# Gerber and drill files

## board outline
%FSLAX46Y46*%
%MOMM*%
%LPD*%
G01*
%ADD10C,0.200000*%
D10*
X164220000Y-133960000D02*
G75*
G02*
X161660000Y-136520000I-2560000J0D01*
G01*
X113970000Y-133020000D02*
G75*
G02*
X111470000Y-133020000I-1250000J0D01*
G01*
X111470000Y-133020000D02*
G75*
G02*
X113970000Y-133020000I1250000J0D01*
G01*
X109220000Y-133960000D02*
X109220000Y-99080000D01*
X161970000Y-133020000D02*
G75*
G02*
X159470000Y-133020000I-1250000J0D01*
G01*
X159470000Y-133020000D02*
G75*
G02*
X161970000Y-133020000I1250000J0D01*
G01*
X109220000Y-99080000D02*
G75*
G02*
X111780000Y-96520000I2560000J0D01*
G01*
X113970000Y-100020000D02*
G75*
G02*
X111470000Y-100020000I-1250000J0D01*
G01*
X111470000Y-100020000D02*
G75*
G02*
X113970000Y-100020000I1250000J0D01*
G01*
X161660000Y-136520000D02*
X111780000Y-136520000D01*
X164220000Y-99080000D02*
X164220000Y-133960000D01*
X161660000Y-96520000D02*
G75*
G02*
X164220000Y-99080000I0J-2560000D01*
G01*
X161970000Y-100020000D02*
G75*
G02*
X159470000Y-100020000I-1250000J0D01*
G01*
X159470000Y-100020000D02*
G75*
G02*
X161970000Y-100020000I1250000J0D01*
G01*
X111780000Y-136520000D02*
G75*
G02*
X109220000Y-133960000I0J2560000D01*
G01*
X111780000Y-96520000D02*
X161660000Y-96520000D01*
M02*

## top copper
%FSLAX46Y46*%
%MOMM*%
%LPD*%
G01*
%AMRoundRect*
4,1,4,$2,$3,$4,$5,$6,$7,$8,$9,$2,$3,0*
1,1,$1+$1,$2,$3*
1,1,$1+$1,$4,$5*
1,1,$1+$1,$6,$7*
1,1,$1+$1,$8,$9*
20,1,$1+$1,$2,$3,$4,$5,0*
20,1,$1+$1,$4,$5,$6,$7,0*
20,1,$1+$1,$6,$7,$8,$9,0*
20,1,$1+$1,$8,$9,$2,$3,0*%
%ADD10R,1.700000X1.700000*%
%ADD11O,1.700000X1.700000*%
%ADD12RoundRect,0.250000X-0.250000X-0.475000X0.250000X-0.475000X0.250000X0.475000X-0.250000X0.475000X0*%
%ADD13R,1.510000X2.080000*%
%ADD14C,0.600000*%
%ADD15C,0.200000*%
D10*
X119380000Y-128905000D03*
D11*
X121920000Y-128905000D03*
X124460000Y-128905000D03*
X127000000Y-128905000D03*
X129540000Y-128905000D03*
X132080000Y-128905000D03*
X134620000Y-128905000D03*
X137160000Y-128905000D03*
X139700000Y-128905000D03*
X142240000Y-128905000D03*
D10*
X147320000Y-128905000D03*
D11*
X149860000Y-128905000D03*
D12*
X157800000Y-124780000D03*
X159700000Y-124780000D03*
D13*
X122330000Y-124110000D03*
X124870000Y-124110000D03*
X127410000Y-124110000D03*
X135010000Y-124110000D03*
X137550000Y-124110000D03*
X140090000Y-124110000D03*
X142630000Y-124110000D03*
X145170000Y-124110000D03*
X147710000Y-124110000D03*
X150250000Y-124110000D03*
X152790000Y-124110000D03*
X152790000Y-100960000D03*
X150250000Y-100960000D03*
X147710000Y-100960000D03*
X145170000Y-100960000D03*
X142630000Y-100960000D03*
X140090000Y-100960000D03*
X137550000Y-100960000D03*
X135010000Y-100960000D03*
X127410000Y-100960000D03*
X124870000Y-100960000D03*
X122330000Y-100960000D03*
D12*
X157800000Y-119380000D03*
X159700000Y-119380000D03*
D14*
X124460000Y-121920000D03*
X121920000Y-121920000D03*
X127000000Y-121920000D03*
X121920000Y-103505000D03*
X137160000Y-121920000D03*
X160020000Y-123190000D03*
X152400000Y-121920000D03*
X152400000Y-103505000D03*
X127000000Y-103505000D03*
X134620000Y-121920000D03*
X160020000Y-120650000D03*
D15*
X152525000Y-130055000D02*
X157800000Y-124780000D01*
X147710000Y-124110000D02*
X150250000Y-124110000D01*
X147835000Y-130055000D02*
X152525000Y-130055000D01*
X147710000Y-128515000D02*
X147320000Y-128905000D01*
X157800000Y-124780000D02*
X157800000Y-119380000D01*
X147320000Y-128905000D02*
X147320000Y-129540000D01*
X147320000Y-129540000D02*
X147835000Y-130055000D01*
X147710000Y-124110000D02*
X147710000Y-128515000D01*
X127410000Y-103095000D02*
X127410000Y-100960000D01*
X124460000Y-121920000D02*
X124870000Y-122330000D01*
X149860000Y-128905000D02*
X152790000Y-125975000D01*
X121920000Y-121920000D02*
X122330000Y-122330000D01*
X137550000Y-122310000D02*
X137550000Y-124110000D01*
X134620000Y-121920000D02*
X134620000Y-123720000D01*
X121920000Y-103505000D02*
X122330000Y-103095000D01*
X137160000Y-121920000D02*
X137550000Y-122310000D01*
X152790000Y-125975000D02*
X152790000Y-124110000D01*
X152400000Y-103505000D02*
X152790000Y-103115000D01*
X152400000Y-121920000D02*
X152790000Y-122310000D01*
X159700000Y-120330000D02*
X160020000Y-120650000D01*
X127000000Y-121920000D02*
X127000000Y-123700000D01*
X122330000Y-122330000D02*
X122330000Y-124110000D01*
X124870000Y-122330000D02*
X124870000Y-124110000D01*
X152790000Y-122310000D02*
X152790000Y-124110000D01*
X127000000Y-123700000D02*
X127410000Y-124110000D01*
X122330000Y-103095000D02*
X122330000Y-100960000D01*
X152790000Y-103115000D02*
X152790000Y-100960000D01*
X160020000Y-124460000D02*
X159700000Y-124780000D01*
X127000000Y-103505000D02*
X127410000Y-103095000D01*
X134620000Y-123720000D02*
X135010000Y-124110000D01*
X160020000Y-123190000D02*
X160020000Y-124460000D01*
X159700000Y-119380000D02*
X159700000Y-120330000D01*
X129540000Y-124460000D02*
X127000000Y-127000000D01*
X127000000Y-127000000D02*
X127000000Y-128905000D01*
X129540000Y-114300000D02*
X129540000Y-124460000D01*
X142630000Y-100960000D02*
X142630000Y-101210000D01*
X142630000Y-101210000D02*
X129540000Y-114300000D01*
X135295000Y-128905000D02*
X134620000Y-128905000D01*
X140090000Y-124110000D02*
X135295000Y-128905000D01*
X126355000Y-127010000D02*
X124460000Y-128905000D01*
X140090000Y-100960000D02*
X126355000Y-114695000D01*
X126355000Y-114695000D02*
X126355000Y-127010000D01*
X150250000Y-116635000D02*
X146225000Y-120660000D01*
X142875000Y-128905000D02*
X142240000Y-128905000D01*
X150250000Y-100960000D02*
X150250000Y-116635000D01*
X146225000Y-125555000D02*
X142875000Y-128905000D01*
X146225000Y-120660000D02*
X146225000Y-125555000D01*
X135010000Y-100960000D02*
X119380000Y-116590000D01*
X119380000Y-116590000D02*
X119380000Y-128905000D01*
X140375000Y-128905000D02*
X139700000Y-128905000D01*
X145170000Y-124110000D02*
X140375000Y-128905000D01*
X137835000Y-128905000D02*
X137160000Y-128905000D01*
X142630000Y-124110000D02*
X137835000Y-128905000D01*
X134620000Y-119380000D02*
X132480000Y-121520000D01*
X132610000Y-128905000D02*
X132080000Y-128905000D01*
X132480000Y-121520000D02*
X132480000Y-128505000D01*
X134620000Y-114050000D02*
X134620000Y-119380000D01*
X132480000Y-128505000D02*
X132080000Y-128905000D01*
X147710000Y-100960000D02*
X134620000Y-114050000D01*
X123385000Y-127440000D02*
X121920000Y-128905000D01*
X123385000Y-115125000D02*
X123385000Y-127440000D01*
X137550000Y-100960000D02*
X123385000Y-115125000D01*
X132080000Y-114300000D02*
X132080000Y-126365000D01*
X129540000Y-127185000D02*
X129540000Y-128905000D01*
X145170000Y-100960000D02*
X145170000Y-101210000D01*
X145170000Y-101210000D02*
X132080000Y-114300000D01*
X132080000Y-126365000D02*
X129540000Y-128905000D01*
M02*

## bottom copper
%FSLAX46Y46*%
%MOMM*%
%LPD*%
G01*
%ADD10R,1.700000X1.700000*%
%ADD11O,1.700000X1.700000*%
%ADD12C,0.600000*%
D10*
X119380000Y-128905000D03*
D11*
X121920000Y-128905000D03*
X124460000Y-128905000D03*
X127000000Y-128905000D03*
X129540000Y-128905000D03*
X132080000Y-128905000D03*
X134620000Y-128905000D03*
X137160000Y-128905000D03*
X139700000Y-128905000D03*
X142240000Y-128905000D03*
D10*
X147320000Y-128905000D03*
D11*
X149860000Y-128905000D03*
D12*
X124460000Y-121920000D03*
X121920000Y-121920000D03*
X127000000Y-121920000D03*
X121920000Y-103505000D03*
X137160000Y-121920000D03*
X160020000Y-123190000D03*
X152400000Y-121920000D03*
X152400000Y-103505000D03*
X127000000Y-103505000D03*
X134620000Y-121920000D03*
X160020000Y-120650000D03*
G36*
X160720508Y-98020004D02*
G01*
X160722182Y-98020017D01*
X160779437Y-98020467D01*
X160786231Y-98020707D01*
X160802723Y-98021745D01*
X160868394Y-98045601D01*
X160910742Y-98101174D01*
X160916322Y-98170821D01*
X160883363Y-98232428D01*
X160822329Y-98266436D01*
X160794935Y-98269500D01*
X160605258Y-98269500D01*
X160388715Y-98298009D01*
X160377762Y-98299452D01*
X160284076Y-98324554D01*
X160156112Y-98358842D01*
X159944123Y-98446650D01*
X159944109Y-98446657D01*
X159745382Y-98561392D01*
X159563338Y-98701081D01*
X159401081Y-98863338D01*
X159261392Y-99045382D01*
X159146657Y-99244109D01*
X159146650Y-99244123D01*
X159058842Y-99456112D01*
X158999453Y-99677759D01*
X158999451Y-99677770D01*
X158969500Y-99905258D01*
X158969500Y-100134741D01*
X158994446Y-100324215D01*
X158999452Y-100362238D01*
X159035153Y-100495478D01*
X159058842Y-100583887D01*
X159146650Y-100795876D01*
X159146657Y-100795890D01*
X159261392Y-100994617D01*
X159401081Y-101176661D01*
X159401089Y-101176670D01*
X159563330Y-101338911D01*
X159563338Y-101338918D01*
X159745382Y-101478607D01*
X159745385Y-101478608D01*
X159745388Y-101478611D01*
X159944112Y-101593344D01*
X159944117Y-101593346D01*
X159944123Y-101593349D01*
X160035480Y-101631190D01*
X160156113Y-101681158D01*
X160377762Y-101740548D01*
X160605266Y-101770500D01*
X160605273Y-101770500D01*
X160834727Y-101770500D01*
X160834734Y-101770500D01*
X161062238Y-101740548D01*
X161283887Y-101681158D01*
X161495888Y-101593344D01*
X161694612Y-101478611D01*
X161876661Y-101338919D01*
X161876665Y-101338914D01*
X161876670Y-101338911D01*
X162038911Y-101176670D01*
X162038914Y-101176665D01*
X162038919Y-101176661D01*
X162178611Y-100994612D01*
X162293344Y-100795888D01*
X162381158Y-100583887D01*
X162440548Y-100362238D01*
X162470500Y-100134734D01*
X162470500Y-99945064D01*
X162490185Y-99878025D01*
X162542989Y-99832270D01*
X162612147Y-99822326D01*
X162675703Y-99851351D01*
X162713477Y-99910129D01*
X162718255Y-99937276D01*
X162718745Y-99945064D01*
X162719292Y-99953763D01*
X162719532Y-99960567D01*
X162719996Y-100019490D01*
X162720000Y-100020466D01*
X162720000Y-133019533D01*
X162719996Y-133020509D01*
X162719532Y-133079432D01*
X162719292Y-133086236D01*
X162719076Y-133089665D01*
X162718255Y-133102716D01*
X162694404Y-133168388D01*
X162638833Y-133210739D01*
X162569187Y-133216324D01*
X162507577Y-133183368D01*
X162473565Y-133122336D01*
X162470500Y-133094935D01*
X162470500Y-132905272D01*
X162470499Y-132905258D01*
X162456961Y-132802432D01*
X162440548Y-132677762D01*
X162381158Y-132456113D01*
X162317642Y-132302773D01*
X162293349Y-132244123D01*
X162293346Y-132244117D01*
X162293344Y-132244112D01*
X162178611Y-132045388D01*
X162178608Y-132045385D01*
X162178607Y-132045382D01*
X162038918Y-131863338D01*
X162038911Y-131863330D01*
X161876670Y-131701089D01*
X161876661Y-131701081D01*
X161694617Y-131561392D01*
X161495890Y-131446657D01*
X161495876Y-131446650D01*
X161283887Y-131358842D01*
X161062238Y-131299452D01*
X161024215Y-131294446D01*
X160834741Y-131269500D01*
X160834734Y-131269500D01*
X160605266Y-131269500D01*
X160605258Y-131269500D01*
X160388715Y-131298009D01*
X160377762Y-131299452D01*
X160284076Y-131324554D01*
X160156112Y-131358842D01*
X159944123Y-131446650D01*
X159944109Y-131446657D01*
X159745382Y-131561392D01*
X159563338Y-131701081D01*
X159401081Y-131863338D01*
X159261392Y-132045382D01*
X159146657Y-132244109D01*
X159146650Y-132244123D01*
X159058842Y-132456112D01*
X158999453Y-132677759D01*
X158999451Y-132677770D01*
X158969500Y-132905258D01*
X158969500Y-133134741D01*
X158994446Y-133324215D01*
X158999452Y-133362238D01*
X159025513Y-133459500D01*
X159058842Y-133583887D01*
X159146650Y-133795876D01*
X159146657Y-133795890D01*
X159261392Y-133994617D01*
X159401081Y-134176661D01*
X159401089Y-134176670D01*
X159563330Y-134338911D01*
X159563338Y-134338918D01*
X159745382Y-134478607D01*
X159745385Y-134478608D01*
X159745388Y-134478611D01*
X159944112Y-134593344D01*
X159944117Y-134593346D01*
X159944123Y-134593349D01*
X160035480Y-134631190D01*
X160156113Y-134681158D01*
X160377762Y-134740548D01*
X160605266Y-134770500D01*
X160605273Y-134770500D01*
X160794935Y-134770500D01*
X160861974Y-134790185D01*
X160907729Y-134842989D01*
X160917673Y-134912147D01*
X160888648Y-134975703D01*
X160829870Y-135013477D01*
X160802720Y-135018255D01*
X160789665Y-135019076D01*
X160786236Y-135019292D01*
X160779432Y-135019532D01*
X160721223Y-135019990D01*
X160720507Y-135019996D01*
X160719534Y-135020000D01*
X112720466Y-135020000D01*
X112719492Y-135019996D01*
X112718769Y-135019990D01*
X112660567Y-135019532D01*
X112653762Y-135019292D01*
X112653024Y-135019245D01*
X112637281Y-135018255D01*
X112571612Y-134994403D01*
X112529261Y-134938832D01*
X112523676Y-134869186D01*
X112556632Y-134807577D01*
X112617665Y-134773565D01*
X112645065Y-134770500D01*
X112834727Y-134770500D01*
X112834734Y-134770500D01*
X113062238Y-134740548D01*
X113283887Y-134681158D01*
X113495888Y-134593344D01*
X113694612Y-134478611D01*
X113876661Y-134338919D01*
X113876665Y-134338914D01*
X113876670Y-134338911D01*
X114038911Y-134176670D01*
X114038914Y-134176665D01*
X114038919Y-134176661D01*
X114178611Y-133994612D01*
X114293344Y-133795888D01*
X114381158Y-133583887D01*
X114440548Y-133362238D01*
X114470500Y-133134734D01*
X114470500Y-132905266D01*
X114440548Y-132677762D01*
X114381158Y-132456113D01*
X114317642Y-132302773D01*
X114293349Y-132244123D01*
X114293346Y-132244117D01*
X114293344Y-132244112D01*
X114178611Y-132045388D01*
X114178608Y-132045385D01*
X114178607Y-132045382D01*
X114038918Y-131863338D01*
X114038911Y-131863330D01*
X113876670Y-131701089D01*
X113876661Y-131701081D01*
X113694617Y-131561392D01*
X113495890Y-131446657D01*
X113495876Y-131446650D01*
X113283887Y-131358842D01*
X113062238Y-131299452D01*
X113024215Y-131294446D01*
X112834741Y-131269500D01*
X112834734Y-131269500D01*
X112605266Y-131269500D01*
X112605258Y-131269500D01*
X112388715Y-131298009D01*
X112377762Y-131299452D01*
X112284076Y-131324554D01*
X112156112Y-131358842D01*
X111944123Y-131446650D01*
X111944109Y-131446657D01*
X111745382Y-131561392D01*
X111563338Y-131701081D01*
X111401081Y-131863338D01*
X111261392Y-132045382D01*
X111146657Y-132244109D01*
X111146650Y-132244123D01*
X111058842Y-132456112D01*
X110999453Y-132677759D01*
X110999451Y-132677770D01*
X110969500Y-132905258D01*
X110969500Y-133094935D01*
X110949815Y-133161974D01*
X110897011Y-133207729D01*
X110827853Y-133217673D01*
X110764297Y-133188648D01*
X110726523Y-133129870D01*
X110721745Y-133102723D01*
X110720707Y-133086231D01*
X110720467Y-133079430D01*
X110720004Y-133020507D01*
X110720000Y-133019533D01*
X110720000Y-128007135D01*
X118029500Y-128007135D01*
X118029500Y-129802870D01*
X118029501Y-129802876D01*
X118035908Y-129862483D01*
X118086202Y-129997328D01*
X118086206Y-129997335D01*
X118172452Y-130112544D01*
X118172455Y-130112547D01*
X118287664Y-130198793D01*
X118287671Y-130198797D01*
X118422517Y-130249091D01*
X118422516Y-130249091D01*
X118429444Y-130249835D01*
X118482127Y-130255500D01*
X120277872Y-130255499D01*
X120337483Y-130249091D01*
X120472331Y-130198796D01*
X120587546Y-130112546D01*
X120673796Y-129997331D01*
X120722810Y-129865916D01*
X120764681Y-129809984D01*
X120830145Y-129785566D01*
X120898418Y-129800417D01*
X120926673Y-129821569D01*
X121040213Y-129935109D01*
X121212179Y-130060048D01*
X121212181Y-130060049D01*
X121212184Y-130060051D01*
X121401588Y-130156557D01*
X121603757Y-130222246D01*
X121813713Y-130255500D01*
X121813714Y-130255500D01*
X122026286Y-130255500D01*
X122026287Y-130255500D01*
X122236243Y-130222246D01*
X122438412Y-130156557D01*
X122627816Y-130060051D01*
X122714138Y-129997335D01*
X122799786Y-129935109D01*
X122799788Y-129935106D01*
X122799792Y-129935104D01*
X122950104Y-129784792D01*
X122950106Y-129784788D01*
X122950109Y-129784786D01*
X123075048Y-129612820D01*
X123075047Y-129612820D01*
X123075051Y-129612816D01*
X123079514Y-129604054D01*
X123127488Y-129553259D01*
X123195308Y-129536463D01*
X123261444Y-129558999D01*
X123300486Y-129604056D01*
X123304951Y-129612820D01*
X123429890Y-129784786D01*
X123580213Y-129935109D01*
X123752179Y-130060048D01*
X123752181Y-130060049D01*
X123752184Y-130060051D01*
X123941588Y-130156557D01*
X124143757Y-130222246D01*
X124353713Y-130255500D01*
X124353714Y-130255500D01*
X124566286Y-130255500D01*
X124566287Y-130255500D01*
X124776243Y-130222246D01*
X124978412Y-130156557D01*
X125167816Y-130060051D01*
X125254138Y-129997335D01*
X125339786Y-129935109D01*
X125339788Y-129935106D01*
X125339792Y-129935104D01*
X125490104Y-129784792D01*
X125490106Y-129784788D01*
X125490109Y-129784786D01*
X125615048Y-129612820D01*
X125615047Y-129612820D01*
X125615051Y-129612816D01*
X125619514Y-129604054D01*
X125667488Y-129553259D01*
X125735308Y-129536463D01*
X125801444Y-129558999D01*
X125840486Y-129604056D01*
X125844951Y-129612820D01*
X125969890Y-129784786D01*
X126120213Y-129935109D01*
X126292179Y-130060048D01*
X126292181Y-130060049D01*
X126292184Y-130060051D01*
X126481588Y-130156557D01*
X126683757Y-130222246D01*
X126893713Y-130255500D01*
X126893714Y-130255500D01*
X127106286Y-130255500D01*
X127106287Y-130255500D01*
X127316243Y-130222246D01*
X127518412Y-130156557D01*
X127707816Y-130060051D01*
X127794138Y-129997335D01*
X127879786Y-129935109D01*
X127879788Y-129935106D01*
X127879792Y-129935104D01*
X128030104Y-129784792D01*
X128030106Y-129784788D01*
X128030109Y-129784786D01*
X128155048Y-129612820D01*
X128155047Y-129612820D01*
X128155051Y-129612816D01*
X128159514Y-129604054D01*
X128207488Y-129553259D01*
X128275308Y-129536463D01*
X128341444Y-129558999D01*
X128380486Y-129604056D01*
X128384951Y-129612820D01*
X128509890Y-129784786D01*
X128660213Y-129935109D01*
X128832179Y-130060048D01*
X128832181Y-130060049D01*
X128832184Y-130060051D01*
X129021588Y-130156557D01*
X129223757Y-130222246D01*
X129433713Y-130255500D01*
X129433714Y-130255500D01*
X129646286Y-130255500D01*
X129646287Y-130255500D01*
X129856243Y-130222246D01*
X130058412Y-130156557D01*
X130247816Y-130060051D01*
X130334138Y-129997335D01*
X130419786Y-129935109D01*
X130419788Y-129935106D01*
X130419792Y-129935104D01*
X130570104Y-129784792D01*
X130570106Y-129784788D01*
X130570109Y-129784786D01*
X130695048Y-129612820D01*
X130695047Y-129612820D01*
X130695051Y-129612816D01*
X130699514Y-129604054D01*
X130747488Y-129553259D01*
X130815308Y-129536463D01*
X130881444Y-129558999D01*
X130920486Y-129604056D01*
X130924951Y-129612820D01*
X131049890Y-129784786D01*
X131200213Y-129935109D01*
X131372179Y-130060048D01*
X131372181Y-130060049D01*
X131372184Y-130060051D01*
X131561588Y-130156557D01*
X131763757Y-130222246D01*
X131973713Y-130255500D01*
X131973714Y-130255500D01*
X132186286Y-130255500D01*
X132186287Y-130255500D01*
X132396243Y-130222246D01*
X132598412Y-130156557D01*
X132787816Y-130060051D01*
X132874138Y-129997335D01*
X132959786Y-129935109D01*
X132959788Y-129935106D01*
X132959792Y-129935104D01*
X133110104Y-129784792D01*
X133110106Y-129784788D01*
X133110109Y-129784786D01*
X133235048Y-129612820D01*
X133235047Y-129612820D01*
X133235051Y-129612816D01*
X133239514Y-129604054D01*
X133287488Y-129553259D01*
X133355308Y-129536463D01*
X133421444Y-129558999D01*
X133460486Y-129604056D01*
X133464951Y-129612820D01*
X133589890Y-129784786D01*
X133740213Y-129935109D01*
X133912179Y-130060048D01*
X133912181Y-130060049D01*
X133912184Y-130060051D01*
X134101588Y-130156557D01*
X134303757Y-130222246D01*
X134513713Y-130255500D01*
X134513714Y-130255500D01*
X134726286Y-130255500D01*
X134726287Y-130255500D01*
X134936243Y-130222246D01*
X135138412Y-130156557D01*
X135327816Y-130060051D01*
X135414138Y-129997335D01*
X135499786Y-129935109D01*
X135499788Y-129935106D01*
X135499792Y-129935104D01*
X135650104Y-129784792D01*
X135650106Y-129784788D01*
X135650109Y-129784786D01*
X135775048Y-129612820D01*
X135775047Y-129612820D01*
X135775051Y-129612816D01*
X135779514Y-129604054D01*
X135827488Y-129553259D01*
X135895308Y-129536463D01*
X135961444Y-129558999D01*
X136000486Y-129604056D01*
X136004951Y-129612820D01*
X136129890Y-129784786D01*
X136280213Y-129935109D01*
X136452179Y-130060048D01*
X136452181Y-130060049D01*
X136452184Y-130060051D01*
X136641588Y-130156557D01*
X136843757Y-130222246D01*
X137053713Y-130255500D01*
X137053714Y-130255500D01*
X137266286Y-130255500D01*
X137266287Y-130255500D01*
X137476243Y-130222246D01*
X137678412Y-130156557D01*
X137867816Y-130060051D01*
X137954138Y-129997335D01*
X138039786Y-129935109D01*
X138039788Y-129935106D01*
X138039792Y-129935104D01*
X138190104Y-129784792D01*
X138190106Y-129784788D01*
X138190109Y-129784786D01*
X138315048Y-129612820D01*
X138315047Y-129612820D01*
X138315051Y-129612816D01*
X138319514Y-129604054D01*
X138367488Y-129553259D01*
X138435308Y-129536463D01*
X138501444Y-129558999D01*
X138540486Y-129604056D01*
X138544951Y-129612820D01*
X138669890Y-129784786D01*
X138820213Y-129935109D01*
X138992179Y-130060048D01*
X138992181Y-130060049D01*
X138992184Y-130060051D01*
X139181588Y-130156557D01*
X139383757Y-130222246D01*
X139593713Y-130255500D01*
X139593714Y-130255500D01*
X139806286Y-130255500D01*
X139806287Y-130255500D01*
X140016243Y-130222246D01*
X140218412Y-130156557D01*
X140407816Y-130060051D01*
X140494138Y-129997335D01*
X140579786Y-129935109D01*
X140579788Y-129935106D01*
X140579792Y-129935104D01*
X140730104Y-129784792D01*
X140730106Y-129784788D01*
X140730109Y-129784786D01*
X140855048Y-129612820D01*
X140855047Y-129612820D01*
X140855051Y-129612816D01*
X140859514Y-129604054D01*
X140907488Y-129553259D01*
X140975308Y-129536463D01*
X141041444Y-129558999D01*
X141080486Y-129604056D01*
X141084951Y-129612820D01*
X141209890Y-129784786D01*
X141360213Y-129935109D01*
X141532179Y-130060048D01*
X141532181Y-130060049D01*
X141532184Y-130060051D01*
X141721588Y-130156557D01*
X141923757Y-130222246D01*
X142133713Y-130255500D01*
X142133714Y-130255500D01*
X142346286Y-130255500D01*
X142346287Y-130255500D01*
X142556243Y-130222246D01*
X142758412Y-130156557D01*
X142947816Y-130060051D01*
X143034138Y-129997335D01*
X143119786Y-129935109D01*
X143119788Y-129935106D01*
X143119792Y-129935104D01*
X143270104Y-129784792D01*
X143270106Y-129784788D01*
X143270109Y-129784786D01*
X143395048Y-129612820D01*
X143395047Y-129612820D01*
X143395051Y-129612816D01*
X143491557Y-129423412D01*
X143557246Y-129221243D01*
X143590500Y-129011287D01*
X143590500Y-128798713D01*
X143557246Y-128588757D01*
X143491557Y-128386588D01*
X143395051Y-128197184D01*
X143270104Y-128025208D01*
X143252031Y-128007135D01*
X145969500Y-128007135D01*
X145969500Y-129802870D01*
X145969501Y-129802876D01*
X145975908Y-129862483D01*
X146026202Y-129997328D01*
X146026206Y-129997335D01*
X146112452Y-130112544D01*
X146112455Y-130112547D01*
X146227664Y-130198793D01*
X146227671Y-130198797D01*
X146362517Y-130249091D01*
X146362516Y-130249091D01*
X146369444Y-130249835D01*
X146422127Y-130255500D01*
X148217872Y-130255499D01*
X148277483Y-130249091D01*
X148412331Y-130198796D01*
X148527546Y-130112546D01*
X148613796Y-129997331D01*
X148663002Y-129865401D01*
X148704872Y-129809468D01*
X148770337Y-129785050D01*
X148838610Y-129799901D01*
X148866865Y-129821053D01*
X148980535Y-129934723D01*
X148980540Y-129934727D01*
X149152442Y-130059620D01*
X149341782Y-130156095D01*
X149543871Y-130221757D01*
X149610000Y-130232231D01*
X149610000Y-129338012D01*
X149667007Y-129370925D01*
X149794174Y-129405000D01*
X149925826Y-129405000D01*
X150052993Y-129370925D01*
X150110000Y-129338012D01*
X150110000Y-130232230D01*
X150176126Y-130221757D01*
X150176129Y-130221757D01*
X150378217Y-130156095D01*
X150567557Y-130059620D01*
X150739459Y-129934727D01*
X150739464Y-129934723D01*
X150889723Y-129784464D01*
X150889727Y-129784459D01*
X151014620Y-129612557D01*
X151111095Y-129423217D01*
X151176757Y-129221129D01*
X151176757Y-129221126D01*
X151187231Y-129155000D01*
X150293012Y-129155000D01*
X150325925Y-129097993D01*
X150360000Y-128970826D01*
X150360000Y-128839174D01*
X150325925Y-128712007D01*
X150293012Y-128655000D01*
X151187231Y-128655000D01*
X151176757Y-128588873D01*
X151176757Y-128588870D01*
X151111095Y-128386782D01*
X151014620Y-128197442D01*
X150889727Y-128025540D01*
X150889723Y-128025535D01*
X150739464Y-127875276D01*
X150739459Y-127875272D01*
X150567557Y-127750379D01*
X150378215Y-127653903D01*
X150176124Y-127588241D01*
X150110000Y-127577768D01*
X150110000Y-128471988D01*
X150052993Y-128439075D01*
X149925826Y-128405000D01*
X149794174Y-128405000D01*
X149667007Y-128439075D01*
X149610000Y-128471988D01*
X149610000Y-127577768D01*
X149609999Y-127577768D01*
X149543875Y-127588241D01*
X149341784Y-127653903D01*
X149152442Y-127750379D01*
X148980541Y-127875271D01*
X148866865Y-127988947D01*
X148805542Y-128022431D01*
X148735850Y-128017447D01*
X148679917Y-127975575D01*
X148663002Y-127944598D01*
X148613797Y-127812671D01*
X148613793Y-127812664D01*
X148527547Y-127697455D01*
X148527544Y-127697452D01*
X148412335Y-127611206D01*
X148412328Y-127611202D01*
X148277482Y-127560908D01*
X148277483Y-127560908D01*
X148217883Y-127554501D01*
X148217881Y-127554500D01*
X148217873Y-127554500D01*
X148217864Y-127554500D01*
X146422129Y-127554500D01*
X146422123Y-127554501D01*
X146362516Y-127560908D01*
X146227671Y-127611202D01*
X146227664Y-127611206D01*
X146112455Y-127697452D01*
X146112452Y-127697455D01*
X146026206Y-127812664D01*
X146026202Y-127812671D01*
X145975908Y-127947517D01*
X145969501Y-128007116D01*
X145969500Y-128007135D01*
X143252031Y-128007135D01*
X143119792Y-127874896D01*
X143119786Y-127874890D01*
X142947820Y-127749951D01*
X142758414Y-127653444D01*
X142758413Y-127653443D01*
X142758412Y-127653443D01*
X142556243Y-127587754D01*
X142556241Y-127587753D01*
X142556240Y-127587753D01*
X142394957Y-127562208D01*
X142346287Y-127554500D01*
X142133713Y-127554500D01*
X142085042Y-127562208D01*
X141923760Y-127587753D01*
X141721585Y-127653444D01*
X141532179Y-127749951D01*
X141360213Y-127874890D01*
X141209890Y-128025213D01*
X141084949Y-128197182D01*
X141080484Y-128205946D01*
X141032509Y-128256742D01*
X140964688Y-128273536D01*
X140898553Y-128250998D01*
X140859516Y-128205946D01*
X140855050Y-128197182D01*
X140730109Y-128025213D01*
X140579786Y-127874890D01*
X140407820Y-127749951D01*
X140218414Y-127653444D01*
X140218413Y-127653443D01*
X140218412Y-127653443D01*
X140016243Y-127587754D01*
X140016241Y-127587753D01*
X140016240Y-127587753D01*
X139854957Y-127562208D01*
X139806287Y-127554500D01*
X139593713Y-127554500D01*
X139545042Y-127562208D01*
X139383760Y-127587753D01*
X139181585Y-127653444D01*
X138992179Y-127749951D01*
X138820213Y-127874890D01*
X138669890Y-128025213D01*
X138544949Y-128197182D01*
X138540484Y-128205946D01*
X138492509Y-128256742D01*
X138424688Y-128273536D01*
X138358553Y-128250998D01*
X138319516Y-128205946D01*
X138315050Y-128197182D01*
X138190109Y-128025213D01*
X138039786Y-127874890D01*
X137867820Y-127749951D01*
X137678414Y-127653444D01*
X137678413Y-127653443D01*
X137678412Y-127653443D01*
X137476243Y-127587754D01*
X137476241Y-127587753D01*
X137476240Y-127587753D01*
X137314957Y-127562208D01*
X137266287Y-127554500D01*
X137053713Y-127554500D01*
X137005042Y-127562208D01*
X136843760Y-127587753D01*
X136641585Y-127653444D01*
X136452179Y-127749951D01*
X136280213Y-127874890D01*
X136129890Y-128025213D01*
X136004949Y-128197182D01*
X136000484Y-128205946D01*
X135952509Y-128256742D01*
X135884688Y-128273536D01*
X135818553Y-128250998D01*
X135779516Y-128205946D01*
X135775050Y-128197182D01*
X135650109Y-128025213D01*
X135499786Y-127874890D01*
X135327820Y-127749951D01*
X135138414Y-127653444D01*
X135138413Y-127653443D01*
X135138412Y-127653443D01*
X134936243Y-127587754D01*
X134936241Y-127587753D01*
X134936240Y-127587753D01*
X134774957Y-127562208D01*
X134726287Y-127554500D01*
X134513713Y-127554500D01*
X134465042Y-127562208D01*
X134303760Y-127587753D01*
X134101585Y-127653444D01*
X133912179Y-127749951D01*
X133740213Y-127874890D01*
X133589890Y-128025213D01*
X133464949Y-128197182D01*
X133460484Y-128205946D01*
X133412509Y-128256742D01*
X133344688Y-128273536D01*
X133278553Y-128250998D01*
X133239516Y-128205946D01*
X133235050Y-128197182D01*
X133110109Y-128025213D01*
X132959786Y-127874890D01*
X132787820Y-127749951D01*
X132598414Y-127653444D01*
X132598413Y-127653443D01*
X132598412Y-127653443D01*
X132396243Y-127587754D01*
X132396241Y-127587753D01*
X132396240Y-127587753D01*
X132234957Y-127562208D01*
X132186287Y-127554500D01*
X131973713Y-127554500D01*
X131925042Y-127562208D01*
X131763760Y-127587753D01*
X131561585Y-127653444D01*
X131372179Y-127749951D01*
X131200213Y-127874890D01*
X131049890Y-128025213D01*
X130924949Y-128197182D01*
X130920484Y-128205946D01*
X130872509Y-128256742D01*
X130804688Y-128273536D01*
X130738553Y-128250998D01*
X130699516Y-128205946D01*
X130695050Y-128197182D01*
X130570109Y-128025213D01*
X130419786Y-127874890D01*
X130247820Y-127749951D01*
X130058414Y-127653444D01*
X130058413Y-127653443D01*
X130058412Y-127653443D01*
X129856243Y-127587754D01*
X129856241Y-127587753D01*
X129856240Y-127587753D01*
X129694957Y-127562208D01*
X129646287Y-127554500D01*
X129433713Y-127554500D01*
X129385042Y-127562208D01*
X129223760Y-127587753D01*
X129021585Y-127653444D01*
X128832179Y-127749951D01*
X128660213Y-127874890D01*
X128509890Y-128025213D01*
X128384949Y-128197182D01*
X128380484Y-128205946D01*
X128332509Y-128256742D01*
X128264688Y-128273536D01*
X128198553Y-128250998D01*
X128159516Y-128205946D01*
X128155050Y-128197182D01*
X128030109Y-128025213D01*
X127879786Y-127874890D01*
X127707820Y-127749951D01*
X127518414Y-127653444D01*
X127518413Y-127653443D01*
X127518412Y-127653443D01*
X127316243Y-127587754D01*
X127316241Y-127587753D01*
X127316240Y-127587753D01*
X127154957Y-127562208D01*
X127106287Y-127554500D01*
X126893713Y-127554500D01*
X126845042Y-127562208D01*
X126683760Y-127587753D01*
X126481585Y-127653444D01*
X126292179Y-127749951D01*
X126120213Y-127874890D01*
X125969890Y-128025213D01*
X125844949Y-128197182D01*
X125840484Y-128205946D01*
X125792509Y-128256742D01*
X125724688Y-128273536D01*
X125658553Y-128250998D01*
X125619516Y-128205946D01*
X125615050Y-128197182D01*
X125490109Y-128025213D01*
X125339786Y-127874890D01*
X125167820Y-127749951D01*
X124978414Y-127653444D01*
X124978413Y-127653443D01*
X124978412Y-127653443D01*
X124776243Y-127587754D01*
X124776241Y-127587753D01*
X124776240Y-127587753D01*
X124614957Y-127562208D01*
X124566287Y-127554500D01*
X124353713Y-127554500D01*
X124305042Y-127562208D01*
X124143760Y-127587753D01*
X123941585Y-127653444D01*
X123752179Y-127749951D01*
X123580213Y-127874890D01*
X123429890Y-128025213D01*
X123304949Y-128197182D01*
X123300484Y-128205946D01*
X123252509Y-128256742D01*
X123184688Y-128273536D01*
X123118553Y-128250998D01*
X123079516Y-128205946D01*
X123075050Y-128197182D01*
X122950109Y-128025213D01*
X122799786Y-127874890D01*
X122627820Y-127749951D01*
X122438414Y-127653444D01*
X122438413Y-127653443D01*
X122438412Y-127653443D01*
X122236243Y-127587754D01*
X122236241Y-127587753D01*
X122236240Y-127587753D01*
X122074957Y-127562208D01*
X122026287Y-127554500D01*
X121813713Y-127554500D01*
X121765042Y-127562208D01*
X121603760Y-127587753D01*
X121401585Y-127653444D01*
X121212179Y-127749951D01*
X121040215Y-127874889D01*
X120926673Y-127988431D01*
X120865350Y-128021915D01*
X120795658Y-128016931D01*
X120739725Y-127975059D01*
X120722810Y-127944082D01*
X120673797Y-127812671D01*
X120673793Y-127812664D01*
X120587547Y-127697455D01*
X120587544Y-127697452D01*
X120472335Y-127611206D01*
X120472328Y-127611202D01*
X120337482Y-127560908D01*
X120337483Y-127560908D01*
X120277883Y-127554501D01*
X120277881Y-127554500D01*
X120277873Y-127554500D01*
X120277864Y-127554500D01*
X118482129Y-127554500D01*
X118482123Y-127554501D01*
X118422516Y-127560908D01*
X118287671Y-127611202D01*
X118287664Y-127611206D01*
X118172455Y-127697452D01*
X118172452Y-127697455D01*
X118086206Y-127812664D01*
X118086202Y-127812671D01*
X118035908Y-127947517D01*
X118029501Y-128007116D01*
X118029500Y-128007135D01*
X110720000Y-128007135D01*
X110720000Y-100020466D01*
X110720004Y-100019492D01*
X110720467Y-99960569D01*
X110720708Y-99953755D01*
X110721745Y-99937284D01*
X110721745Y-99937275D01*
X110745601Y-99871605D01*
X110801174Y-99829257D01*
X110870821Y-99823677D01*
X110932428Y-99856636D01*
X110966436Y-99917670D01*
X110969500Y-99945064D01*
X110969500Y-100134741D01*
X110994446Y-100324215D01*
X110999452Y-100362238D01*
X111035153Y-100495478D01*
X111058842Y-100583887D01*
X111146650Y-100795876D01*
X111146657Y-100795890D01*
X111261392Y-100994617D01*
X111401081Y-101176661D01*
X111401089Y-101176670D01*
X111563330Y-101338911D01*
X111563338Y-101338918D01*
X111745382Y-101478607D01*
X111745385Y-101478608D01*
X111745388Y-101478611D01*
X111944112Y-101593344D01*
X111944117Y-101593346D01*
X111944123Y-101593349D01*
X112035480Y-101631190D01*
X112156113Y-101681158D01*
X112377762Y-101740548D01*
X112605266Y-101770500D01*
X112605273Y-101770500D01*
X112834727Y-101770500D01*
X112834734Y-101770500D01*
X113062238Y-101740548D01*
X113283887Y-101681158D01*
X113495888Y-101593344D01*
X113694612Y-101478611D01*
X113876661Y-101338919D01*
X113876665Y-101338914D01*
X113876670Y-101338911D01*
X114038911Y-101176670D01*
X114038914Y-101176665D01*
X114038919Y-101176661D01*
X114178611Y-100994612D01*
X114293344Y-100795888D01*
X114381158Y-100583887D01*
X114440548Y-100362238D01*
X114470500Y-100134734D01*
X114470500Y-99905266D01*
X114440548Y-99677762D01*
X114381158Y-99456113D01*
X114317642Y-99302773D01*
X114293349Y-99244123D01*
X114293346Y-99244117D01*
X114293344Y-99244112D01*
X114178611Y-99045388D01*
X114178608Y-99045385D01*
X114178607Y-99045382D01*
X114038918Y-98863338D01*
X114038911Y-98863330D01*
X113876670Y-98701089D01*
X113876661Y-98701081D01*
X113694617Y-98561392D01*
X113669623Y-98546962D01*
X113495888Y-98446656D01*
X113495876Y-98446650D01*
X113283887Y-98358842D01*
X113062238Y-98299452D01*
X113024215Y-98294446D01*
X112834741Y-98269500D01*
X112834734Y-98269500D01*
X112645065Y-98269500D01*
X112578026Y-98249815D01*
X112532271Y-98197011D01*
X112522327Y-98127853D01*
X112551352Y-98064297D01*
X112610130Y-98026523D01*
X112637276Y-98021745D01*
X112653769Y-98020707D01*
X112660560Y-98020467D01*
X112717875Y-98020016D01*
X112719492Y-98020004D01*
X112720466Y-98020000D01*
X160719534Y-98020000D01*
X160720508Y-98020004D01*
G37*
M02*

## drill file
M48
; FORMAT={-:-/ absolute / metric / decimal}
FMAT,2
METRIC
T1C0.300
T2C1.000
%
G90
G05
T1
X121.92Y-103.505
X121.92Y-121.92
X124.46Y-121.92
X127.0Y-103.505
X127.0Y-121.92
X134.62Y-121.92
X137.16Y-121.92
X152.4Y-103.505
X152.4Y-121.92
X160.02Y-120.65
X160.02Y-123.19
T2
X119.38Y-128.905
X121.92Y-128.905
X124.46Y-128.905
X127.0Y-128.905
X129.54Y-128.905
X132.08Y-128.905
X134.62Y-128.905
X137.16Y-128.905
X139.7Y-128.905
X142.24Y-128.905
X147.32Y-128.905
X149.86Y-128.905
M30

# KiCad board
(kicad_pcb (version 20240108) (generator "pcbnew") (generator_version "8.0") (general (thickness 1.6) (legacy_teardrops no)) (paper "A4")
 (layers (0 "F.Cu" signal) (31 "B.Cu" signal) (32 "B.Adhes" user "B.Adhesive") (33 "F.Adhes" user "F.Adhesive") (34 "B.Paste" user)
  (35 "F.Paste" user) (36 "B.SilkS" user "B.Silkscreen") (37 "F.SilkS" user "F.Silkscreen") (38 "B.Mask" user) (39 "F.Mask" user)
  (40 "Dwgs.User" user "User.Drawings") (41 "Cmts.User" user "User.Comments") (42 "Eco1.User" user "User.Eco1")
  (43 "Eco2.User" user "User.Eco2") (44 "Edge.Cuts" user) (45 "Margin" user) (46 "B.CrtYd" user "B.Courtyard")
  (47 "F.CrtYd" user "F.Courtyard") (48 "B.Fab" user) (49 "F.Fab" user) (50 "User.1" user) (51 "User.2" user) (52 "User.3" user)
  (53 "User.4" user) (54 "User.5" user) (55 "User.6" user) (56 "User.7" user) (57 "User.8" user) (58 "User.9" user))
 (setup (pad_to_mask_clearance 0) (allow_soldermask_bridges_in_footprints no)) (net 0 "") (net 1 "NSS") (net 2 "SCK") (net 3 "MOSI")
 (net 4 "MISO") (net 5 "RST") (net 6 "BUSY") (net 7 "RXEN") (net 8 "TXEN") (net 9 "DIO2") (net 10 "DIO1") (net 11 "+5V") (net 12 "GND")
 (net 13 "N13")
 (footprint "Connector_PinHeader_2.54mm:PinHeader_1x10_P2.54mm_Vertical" (layer "F.Cu") (at 119.38 128.905 90)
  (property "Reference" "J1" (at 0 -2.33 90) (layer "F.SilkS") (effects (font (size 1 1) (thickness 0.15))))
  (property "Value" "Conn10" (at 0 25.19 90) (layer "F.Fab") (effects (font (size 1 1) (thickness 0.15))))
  (pad "1" thru_hole rect (at 0 0 90) (size 1.7 1.7) (drill 1) (layers "*.Cu" "*.Mask") (remove_unused_layers no) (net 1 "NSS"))
  (pad "2" thru_hole oval (at 0 2.54 90) (size 1.7 1.7) (drill 1) (layers "*.Cu" "*.Mask") (remove_unused_layers no) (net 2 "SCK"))
  (pad "3" thru_hole oval (at 0 5.08 90) (size 1.7 1.7) (drill 1) (layers "*.Cu" "*.Mask") (remove_unused_layers no) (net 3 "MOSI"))
  (pad "4" thru_hole oval (at 0 7.62 90) (size 1.7 1.7) (drill 1) (layers "*.Cu" "*.Mask") (remove_unused_layers no) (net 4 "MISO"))
  (pad "5" thru_hole oval (at 0 10.16 90) (size 1.7 1.7) (drill 1) (layers "*.Cu" "*.Mask") (remove_unused_layers no) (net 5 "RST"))
  (pad "6" thru_hole oval (at 0 12.7 90) (size 1.7 1.7) (drill 1) (layers "*.Cu" "*.Mask") (remove_unused_layers no) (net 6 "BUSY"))
  (pad "7" thru_hole oval (at 0 15.24 90) (size 1.7 1.7) (drill 1) (layers "*.Cu" "*.Mask") (remove_unused_layers no) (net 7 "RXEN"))
  (pad "8" thru_hole oval (at 0 17.78 90) (size 1.7 1.7) (drill 1) (layers "*.Cu" "*.Mask") (remove_unused_layers no) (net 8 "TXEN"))
  (pad "9" thru_hole oval (at 0 20.32 90) (size 1.7 1.7) (drill 1) (layers "*.Cu" "*.Mask") (remove_unused_layers no) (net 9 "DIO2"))
  (pad "10" thru_hole oval (at 0 22.86 90) (size 1.7 1.7) (drill 1) (layers "*.Cu" "*.Mask") (remove_unused_layers no) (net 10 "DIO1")))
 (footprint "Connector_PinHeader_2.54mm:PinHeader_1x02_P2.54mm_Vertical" (layer "F.Cu") (at 147.32 128.905 90)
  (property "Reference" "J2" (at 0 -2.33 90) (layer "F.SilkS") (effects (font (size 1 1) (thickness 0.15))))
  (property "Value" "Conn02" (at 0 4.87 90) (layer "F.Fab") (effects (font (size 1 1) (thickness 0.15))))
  (pad "1" thru_hole rect (at 0 0 90) (size 1.7 1.7) (drill 1) (layers "*.Cu" "*.Mask") (remove_unused_layers no) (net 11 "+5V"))
  (pad "2" thru_hole oval (at 0 2.54 90) (size 1.7 1.7) (drill 1) (layers "*.Cu" "*.Mask") (remove_unused_layers no) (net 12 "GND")))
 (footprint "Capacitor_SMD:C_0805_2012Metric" (layer "F.Cu") (at 158.75 124.78)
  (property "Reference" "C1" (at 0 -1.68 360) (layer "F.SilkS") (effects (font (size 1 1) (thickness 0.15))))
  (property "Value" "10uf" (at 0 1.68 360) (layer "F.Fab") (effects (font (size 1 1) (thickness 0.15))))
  (pad "1" smd roundrect (at -0.95 0) (size 1 1.45) (layers "F.Cu" "F.Paste" "F.Mask") (roundrect_rratio 0.25) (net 11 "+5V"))
  (pad "2" smd roundrect (at 0.95 0) (size 1 1.45) (layers "F.Cu" "F.Paste" "F.Mask") (roundrect_rratio 0.25) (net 12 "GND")))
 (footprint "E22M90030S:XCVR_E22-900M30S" (layer "F.Cu") (at 136.15 112.535 -90)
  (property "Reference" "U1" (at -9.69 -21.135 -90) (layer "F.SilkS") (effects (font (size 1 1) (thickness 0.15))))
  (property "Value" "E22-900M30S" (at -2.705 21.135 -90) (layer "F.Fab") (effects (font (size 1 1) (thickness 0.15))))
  (pad "1" smd rect (at 11.575 13.82 270) (size 2.08 1.51) (layers "F.Cu" "F.Paste" "F.Mask") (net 12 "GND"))
  (pad "2" smd rect (at 11.575 11.28 270) (size 2.08 1.51) (layers "F.Cu" "F.Paste" "F.Mask") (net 12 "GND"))
  (pad "3" smd rect (at 11.575 8.74 270) (size 2.08 1.51) (layers "F.Cu" "F.Paste" "F.Mask") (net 12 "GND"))
  (pad "4" smd rect (at 11.575 1.14 270) (size 2.08 1.51) (layers "F.Cu" "F.Paste" "F.Mask") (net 12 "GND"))
  (pad "5" smd rect (at 11.575 -1.4 270) (size 2.08 1.51) (layers "F.Cu" "F.Paste" "F.Mask") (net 12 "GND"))
  (pad "6" smd rect (at 11.575 -3.94 270) (size 2.08 1.51) (layers "F.Cu" "F.Paste" "F.Mask") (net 7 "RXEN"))
  (pad "7" smd rect (at 11.575 -6.48 270) (size 2.08 1.51) (layers "F.Cu" "F.Paste" "F.Mask") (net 8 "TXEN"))
  (pad "8" smd rect (at 11.575 -9.02 270) (size 2.08 1.51) (layers "F.Cu" "F.Paste" "F.Mask") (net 9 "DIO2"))
  (pad "9" smd rect (at 11.575 -11.56 270) (size 2.08 1.51) (layers "F.Cu" "F.Paste" "F.Mask") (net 11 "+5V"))
  (pad "10" smd rect (at 11.575 -14.1 270) (size 2.08 1.51) (layers "F.Cu" "F.Paste" "F.Mask") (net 11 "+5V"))
  (pad "11" smd rect (at 11.575 -16.64 270) (size 2.08 1.51) (layers "F.Cu" "F.Paste" "F.Mask") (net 12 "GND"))
  (pad "12" smd rect (at -11.575 -16.64 270) (size 2.08 1.51) (layers "F.Cu" "F.Paste" "F.Mask") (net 12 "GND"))
  (pad "13" smd rect (at -11.575 -14.1 270) (size 2.08 1.51) (layers "F.Cu" "F.Paste" "F.Mask") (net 10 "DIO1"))
  (pad "14" smd rect (at -11.575 -11.56 270) (size 2.08 1.51) (layers "F.Cu" "F.Paste" "F.Mask") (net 6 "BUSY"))
  (pad "15" smd rect (at -11.575 -9.02 270) (size 2.08 1.51) (layers "F.Cu" "F.Paste" "F.Mask") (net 5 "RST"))
  (pad "16" smd rect (at -11.575 -6.48 270) (size 2.08 1.51) (layers "F.Cu" "F.Paste" "F.Mask") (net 4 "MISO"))
  (pad "17" smd rect (at -11.575 -3.94 270) (size 2.08 1.51) (layers "F.Cu" "F.Paste" "F.Mask") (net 3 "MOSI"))
  (pad "18" smd rect (at -11.575 -1.4 270) (size 2.08 1.51) (layers "F.Cu" "F.Paste" "F.Mask") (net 2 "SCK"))
  (pad "19" smd rect (at -11.575 1.14 270) (size 2.08 1.51) (layers "F.Cu" "F.Paste" "F.Mask") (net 1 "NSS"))
  (pad "20" smd rect (at -11.575 8.74 270) (size 2.08 1.51) (layers "F.Cu" "F.Paste" "F.Mask") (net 12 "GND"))
  (pad "21" smd rect (at -11.575 11.28 270) (size 2.08 1.51) (layers "F.Cu" "F.Paste" "F.Mask") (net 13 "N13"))
  (pad "22" smd rect (at -11.575 13.82 270) (size 2.08 1.51) (layers "F.Cu" "F.Paste" "F.Mask") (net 12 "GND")))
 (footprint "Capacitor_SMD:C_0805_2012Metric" (layer "F.Cu") (at 158.75 119.38)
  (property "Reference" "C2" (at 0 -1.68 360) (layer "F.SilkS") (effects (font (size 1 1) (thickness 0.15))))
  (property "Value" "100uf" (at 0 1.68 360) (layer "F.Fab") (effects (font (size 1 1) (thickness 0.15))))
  (pad "1" smd roundrect (at -0.95 0) (size 1 1.45) (layers "F.Cu" "F.Paste" "F.Mask") (roundrect_rratio 0.25) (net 11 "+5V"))
  (pad "2" smd roundrect (at 0.95 0) (size 1 1.45) (layers "F.Cu" "F.Paste" "F.Mask") (roundrect_rratio 0.25) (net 12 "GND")))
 (gr_arc (start 164.22 133.96) (mid 163.470193 135.770193) (end 161.66 136.52) (stroke (width 0.2) (type default)) (layer "Edge.Cuts"))
 (gr_circle (center 112.72 133.02) (end 113.97 133.02) (stroke (width 0.2) (type default)) (fill none) (layer "Edge.Cuts"))
 (gr_line (start 109.22 133.96) (end 109.22 99.08) (stroke (width 0.2) (type default)) (layer "Edge.Cuts"))
 (gr_circle (center 160.72 133.02) (end 161.97 133.02) (stroke (width 0.2) (type default)) (fill none) (layer "Edge.Cuts"))
 (gr_arc (start 109.22 99.08) (mid 109.969807 97.269807) (end 111.78 96.52) (stroke (width 0.2) (type default)) (layer "Edge.Cuts"))
 (gr_circle (center 112.72 100.02) (end 113.97 100.02) (stroke (width 0.2) (type default)) (fill none) (layer "Edge.Cuts"))
 (gr_line (start 161.66 136.52) (end 111.78 136.52) (stroke (width 0.2) (type default)) (layer "Edge.Cuts"))
 (gr_line (start 164.22 99.08) (end 164.22 133.96) (stroke (width 0.2) (type default)) (layer "Edge.Cuts"))
 (gr_arc (start 161.66 96.52) (mid 163.470193 97.269807) (end 164.22 99.08) (stroke (width 0.2) (type default)) (layer "Edge.Cuts"))
 (gr_circle (center 160.72 100.02) (end 161.97 100.02) (stroke (width 0.2) (type default)) (fill none) (layer "Edge.Cuts"))
 (gr_arc (start 111.78 136.52) (mid 109.969807 135.770193) (end 109.22 133.96) (stroke (width 0.2) (type default)) (layer "Edge.Cuts"))
 (gr_line (start 111.78 96.52) (end 161.66 96.52) (stroke (width 0.2) (type default)) (layer "Edge.Cuts"))
 (segment (start 152.525 130.055) (end 157.8 124.78) (width 0.2) (layer "F.Cu") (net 11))
 (segment (start 147.71 124.11) (end 150.25 124.11) (width 0.2) (layer "F.Cu") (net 11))
 (segment (start 147.835 130.055) (end 152.525 130.055) (width 0.2) (layer "F.Cu") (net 11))
 (segment (start 147.71 128.515) (end 147.32 128.905) (width 0.2) (layer "F.Cu") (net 11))
 (segment (start 157.8 124.78) (end 157.8 119.38) (width 0.2) (layer "F.Cu") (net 11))
 (segment (start 147.32 128.905) (end 147.32 129.54) (width 0.2) (layer "F.Cu") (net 11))
 (segment (start 147.32 129.54) (end 147.835 130.055) (width 0.2) (layer "F.Cu") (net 11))
 (segment (start 147.71 124.11) (end 147.71 128.515) (width 0.2) (layer "F.Cu") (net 11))
 (segment (start 127.41 103.095) (end 127.41 100.96) (width 0.2) (layer "F.Cu") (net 12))
 (segment (start 124.46 121.92) (end 124.87 122.33) (width 0.2) (layer "F.Cu") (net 12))
 (segment (start 149.86 128.905) (end 152.79 125.975) (width 0.2) (layer "F.Cu") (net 12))
 (segment (start 121.92 121.92) (end 122.33 122.33) (width 0.2) (layer "F.Cu") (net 12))
 (segment (start 137.55 122.31) (end 137.55 124.11) (width 0.2) (layer "F.Cu") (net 12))
 (segment (start 134.62 121.92) (end 134.62 123.72) (width 0.2) (layer "F.Cu") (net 12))
 (segment (start 121.92 103.505) (end 122.33 103.095) (width 0.2) (layer "F.Cu") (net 12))
 (segment (start 137.16 121.92) (end 137.55 122.31) (width 0.2) (layer "F.Cu") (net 12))
 (segment (start 152.79 125.975) (end 152.79 124.11) (width 0.2) (layer "F.Cu") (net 12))
 (segment (start 152.4 103.505) (end 152.79 103.115) (width 0.2) (layer "F.Cu") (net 12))
 (segment (start 152.4 121.92) (end 152.79 122.31) (width 0.2) (layer "F.Cu") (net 12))
 (segment (start 159.7 120.33) (end 160.02 120.65) (width 0.2) (layer "F.Cu") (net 12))
 (segment (start 127 121.92) (end 127 123.7) (width 0.2) (layer "F.Cu") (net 12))
 (segment (start 122.33 122.33) (end 122.33 124.11) (width 0.2) (layer "F.Cu") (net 12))
 (segment (start 124.87 122.33) (end 124.87 124.11) (width 0.2) (layer "F.Cu") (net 12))
 (segment (start 152.79 122.31) (end 152.79 124.11) (width 0.2) (layer "F.Cu") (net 12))
 (segment (start 127 123.7) (end 127.41 124.11) (width 0.2) (layer "F.Cu") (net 12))
 (segment (start 122.33 103.095) (end 122.33 100.96) (width 0.2) (layer "F.Cu") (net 12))
 (segment (start 152.79 103.115) (end 152.79 100.96) (width 0.2) (layer "F.Cu") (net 12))
 (segment (start 160.02 124.46) (end 159.7 124.78) (width 0.2) (layer "F.Cu") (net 12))
 (segment (start 127 103.505) (end 127.41 103.095) (width 0.2) (layer "F.Cu") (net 12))
 (segment (start 134.62 123.72) (end 135.01 124.11) (width 0.2) (layer "F.Cu") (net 12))
 (segment (start 160.02 123.19) (end 160.02 124.46) (width 0.2) (layer "F.Cu") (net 12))
 (segment (start 159.7 119.38) (end 159.7 120.33) (width 0.2) (layer "F.Cu") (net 12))
 (via (at 124.46 121.92) (size 0.6) (drill 0.3) (layers "F.Cu" "B.Cu") (free yes) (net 12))
 (via (at 121.92 121.92) (size 0.6) (drill 0.3) (layers "F.Cu" "B.Cu") (free yes) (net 12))
 (via (at 127 121.92) (size 0.6) (drill 0.3) (layers "F.Cu" "B.Cu") (free yes) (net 12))
 (via (at 121.92 103.505) (size 0.6) (drill 0.3) (layers "F.Cu" "B.Cu") (free yes) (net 12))
 (via (at 137.16 121.92) (size 0.6) (drill 0.3) (layers "F.Cu" "B.Cu") (free yes) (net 12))
 (via (at 160.02 123.19) (size 0.6) (drill 0.3) (layers "F.Cu" "B.Cu") (free yes) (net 12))
 (via (at 152.4 121.92) (size 0.6) (drill 0.3) (layers "F.Cu" "B.Cu") (free yes) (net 12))
 (via (at 152.4 103.505) (size 0.6) (drill 0.3) (layers "F.Cu" "B.Cu") (free yes) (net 12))
 (via (at 127 103.505) (size 0.6) (drill 0.3) (layers "F.Cu" "B.Cu") (free yes) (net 12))
 (via (at 134.62 121.92) (size 0.6) (drill 0.3) (layers "F.Cu" "B.Cu") (free yes) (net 12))
 (via (at 160.02 120.65) (size 0.6) (drill 0.3) (layers "F.Cu" "B.Cu") (free yes) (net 12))
 (segment (start 129.54 124.46) (end 127 127) (width 0.2) (layer "F.Cu") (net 4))
 (segment (start 127 127) (end 127 128.905) (width 0.2) (layer "F.Cu") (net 4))
 (segment (start 129.54 114.3) (end 129.54 124.46) (width 0.2) (layer "F.Cu") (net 4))
 (segment (start 142.63 100.96) (end 142.63 101.21) (width 0.2) (layer "F.Cu") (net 4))
 (segment (start 142.63 101.21) (end 129.54 114.3) (width 0.2) (layer "F.Cu") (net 4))
 (segment (start 135.295 128.905) (end 134.62 128.905) (width 0.2) (layer "F.Cu") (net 7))
 (segment (start 140.09 124.11) (end 135.295 128.905) (width 0.2) (layer "F.Cu") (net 7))
 (segment (start 126.355 127.01) (end 124.46 128.905) (width 0.2) (layer "F.Cu") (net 3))
 (segment (start 140.09 100.96) (end 126.355 114.695) (width 0.2) (layer "F.Cu") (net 3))
 (segment (start 126.355 114.695) (end 126.355 127.01) (width 0.2) (layer "F.Cu") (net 3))
 (segment (start 150.25 116.635) (end 146.225 120.66) (width 0.2) (layer "F.Cu") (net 10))
 (segment (start 142.875 128.905) (end 142.24 128.905) (width 0.2) (layer "F.Cu") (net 10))
 (segment (start 150.25 100.96) (end 150.25 116.635) (width 0.2) (layer "F.Cu") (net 10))
 (segment (start 146.225 125.555) (end 142.875 128.905) (width 0.2) (layer "F.Cu") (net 10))
 (segment (start 146.225 120.66) (end 146.225 125.555) (width 0.2) (layer "F.Cu") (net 10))
 (segment (start 135.01 100.96) (end 119.38 116.59) (width 0.2) (layer "F.Cu") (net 1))
 (segment (start 119.38 116.59) (end 119.38 128.905) (width 0.2) (layer "F.Cu") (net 1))
 (segment (start 140.375 128.905) (end 139.7 128.905) (width 0.2) (layer "F.Cu") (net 9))
 (segment (start 145.17 124.11) (end 140.375 128.905) (width 0.2) (layer "F.Cu") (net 9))
 (segment (start 137.835 128.905) (end 137.16 128.905) (width 0.2) (layer "F.Cu") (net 8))
 (segment (start 142.63 124.11) (end 137.835 128.905) (width 0.2) (layer "F.Cu") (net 8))
 (segment (start 134.62 119.38) (end 132.48 121.52) (width 0.2) (layer "F.Cu") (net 6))
 (segment (start 132.61 128.905) (end 132.08 128.905) (width 0.2) (layer "F.Cu") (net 6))
 (segment (start 132.48 121.52) (end 132.48 128.505) (width 0.2) (layer "F.Cu") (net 6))
 (segment (start 134.62 114.05) (end 134.62 119.38) (width 0.2) (layer "F.Cu") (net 6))
 (segment (start 132.48 128.505) (end 132.08 128.905) (width 0.2) (layer "F.Cu") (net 6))
 (segment (start 147.71 100.96) (end 134.62 114.05) (width 0.2) (layer "F.Cu") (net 6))
 (segment (start 123.385 127.44) (end 121.92 128.905) (width 0.2) (layer "F.Cu") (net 2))
 (segment (start 123.385 115.125) (end 123.385 127.44) (width 0.2) (layer "F.Cu") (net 2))
 (segment (start 137.55 100.96) (end 123.385 115.125) (width 0.2) (layer "F.Cu") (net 2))
 (segment (start 132.08 114.3) (end 132.08 126.365) (width 0.2) (layer "F.Cu") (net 5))
 (segment (start 129.54 127.185) (end 129.54 128.905) (width 0.2) (layer "F.Cu") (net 5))
 (segment (start 145.17 100.96) (end 145.17 101.21) (width 0.2) (layer "F.Cu") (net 5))
 (segment (start 145.17 101.21) (end 132.08 114.3) (width 0.2) (layer "F.Cu") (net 5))
 (segment (start 132.08 126.365) (end 129.54 128.905) (width 0.2) (layer "F.Cu") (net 5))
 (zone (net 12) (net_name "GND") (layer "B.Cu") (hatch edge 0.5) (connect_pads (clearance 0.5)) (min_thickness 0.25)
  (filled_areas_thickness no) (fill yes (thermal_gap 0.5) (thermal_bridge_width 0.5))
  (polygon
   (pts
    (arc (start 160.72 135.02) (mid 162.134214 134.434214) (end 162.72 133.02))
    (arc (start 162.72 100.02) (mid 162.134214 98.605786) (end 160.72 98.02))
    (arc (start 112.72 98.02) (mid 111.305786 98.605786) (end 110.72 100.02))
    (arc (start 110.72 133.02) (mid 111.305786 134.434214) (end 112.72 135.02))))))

